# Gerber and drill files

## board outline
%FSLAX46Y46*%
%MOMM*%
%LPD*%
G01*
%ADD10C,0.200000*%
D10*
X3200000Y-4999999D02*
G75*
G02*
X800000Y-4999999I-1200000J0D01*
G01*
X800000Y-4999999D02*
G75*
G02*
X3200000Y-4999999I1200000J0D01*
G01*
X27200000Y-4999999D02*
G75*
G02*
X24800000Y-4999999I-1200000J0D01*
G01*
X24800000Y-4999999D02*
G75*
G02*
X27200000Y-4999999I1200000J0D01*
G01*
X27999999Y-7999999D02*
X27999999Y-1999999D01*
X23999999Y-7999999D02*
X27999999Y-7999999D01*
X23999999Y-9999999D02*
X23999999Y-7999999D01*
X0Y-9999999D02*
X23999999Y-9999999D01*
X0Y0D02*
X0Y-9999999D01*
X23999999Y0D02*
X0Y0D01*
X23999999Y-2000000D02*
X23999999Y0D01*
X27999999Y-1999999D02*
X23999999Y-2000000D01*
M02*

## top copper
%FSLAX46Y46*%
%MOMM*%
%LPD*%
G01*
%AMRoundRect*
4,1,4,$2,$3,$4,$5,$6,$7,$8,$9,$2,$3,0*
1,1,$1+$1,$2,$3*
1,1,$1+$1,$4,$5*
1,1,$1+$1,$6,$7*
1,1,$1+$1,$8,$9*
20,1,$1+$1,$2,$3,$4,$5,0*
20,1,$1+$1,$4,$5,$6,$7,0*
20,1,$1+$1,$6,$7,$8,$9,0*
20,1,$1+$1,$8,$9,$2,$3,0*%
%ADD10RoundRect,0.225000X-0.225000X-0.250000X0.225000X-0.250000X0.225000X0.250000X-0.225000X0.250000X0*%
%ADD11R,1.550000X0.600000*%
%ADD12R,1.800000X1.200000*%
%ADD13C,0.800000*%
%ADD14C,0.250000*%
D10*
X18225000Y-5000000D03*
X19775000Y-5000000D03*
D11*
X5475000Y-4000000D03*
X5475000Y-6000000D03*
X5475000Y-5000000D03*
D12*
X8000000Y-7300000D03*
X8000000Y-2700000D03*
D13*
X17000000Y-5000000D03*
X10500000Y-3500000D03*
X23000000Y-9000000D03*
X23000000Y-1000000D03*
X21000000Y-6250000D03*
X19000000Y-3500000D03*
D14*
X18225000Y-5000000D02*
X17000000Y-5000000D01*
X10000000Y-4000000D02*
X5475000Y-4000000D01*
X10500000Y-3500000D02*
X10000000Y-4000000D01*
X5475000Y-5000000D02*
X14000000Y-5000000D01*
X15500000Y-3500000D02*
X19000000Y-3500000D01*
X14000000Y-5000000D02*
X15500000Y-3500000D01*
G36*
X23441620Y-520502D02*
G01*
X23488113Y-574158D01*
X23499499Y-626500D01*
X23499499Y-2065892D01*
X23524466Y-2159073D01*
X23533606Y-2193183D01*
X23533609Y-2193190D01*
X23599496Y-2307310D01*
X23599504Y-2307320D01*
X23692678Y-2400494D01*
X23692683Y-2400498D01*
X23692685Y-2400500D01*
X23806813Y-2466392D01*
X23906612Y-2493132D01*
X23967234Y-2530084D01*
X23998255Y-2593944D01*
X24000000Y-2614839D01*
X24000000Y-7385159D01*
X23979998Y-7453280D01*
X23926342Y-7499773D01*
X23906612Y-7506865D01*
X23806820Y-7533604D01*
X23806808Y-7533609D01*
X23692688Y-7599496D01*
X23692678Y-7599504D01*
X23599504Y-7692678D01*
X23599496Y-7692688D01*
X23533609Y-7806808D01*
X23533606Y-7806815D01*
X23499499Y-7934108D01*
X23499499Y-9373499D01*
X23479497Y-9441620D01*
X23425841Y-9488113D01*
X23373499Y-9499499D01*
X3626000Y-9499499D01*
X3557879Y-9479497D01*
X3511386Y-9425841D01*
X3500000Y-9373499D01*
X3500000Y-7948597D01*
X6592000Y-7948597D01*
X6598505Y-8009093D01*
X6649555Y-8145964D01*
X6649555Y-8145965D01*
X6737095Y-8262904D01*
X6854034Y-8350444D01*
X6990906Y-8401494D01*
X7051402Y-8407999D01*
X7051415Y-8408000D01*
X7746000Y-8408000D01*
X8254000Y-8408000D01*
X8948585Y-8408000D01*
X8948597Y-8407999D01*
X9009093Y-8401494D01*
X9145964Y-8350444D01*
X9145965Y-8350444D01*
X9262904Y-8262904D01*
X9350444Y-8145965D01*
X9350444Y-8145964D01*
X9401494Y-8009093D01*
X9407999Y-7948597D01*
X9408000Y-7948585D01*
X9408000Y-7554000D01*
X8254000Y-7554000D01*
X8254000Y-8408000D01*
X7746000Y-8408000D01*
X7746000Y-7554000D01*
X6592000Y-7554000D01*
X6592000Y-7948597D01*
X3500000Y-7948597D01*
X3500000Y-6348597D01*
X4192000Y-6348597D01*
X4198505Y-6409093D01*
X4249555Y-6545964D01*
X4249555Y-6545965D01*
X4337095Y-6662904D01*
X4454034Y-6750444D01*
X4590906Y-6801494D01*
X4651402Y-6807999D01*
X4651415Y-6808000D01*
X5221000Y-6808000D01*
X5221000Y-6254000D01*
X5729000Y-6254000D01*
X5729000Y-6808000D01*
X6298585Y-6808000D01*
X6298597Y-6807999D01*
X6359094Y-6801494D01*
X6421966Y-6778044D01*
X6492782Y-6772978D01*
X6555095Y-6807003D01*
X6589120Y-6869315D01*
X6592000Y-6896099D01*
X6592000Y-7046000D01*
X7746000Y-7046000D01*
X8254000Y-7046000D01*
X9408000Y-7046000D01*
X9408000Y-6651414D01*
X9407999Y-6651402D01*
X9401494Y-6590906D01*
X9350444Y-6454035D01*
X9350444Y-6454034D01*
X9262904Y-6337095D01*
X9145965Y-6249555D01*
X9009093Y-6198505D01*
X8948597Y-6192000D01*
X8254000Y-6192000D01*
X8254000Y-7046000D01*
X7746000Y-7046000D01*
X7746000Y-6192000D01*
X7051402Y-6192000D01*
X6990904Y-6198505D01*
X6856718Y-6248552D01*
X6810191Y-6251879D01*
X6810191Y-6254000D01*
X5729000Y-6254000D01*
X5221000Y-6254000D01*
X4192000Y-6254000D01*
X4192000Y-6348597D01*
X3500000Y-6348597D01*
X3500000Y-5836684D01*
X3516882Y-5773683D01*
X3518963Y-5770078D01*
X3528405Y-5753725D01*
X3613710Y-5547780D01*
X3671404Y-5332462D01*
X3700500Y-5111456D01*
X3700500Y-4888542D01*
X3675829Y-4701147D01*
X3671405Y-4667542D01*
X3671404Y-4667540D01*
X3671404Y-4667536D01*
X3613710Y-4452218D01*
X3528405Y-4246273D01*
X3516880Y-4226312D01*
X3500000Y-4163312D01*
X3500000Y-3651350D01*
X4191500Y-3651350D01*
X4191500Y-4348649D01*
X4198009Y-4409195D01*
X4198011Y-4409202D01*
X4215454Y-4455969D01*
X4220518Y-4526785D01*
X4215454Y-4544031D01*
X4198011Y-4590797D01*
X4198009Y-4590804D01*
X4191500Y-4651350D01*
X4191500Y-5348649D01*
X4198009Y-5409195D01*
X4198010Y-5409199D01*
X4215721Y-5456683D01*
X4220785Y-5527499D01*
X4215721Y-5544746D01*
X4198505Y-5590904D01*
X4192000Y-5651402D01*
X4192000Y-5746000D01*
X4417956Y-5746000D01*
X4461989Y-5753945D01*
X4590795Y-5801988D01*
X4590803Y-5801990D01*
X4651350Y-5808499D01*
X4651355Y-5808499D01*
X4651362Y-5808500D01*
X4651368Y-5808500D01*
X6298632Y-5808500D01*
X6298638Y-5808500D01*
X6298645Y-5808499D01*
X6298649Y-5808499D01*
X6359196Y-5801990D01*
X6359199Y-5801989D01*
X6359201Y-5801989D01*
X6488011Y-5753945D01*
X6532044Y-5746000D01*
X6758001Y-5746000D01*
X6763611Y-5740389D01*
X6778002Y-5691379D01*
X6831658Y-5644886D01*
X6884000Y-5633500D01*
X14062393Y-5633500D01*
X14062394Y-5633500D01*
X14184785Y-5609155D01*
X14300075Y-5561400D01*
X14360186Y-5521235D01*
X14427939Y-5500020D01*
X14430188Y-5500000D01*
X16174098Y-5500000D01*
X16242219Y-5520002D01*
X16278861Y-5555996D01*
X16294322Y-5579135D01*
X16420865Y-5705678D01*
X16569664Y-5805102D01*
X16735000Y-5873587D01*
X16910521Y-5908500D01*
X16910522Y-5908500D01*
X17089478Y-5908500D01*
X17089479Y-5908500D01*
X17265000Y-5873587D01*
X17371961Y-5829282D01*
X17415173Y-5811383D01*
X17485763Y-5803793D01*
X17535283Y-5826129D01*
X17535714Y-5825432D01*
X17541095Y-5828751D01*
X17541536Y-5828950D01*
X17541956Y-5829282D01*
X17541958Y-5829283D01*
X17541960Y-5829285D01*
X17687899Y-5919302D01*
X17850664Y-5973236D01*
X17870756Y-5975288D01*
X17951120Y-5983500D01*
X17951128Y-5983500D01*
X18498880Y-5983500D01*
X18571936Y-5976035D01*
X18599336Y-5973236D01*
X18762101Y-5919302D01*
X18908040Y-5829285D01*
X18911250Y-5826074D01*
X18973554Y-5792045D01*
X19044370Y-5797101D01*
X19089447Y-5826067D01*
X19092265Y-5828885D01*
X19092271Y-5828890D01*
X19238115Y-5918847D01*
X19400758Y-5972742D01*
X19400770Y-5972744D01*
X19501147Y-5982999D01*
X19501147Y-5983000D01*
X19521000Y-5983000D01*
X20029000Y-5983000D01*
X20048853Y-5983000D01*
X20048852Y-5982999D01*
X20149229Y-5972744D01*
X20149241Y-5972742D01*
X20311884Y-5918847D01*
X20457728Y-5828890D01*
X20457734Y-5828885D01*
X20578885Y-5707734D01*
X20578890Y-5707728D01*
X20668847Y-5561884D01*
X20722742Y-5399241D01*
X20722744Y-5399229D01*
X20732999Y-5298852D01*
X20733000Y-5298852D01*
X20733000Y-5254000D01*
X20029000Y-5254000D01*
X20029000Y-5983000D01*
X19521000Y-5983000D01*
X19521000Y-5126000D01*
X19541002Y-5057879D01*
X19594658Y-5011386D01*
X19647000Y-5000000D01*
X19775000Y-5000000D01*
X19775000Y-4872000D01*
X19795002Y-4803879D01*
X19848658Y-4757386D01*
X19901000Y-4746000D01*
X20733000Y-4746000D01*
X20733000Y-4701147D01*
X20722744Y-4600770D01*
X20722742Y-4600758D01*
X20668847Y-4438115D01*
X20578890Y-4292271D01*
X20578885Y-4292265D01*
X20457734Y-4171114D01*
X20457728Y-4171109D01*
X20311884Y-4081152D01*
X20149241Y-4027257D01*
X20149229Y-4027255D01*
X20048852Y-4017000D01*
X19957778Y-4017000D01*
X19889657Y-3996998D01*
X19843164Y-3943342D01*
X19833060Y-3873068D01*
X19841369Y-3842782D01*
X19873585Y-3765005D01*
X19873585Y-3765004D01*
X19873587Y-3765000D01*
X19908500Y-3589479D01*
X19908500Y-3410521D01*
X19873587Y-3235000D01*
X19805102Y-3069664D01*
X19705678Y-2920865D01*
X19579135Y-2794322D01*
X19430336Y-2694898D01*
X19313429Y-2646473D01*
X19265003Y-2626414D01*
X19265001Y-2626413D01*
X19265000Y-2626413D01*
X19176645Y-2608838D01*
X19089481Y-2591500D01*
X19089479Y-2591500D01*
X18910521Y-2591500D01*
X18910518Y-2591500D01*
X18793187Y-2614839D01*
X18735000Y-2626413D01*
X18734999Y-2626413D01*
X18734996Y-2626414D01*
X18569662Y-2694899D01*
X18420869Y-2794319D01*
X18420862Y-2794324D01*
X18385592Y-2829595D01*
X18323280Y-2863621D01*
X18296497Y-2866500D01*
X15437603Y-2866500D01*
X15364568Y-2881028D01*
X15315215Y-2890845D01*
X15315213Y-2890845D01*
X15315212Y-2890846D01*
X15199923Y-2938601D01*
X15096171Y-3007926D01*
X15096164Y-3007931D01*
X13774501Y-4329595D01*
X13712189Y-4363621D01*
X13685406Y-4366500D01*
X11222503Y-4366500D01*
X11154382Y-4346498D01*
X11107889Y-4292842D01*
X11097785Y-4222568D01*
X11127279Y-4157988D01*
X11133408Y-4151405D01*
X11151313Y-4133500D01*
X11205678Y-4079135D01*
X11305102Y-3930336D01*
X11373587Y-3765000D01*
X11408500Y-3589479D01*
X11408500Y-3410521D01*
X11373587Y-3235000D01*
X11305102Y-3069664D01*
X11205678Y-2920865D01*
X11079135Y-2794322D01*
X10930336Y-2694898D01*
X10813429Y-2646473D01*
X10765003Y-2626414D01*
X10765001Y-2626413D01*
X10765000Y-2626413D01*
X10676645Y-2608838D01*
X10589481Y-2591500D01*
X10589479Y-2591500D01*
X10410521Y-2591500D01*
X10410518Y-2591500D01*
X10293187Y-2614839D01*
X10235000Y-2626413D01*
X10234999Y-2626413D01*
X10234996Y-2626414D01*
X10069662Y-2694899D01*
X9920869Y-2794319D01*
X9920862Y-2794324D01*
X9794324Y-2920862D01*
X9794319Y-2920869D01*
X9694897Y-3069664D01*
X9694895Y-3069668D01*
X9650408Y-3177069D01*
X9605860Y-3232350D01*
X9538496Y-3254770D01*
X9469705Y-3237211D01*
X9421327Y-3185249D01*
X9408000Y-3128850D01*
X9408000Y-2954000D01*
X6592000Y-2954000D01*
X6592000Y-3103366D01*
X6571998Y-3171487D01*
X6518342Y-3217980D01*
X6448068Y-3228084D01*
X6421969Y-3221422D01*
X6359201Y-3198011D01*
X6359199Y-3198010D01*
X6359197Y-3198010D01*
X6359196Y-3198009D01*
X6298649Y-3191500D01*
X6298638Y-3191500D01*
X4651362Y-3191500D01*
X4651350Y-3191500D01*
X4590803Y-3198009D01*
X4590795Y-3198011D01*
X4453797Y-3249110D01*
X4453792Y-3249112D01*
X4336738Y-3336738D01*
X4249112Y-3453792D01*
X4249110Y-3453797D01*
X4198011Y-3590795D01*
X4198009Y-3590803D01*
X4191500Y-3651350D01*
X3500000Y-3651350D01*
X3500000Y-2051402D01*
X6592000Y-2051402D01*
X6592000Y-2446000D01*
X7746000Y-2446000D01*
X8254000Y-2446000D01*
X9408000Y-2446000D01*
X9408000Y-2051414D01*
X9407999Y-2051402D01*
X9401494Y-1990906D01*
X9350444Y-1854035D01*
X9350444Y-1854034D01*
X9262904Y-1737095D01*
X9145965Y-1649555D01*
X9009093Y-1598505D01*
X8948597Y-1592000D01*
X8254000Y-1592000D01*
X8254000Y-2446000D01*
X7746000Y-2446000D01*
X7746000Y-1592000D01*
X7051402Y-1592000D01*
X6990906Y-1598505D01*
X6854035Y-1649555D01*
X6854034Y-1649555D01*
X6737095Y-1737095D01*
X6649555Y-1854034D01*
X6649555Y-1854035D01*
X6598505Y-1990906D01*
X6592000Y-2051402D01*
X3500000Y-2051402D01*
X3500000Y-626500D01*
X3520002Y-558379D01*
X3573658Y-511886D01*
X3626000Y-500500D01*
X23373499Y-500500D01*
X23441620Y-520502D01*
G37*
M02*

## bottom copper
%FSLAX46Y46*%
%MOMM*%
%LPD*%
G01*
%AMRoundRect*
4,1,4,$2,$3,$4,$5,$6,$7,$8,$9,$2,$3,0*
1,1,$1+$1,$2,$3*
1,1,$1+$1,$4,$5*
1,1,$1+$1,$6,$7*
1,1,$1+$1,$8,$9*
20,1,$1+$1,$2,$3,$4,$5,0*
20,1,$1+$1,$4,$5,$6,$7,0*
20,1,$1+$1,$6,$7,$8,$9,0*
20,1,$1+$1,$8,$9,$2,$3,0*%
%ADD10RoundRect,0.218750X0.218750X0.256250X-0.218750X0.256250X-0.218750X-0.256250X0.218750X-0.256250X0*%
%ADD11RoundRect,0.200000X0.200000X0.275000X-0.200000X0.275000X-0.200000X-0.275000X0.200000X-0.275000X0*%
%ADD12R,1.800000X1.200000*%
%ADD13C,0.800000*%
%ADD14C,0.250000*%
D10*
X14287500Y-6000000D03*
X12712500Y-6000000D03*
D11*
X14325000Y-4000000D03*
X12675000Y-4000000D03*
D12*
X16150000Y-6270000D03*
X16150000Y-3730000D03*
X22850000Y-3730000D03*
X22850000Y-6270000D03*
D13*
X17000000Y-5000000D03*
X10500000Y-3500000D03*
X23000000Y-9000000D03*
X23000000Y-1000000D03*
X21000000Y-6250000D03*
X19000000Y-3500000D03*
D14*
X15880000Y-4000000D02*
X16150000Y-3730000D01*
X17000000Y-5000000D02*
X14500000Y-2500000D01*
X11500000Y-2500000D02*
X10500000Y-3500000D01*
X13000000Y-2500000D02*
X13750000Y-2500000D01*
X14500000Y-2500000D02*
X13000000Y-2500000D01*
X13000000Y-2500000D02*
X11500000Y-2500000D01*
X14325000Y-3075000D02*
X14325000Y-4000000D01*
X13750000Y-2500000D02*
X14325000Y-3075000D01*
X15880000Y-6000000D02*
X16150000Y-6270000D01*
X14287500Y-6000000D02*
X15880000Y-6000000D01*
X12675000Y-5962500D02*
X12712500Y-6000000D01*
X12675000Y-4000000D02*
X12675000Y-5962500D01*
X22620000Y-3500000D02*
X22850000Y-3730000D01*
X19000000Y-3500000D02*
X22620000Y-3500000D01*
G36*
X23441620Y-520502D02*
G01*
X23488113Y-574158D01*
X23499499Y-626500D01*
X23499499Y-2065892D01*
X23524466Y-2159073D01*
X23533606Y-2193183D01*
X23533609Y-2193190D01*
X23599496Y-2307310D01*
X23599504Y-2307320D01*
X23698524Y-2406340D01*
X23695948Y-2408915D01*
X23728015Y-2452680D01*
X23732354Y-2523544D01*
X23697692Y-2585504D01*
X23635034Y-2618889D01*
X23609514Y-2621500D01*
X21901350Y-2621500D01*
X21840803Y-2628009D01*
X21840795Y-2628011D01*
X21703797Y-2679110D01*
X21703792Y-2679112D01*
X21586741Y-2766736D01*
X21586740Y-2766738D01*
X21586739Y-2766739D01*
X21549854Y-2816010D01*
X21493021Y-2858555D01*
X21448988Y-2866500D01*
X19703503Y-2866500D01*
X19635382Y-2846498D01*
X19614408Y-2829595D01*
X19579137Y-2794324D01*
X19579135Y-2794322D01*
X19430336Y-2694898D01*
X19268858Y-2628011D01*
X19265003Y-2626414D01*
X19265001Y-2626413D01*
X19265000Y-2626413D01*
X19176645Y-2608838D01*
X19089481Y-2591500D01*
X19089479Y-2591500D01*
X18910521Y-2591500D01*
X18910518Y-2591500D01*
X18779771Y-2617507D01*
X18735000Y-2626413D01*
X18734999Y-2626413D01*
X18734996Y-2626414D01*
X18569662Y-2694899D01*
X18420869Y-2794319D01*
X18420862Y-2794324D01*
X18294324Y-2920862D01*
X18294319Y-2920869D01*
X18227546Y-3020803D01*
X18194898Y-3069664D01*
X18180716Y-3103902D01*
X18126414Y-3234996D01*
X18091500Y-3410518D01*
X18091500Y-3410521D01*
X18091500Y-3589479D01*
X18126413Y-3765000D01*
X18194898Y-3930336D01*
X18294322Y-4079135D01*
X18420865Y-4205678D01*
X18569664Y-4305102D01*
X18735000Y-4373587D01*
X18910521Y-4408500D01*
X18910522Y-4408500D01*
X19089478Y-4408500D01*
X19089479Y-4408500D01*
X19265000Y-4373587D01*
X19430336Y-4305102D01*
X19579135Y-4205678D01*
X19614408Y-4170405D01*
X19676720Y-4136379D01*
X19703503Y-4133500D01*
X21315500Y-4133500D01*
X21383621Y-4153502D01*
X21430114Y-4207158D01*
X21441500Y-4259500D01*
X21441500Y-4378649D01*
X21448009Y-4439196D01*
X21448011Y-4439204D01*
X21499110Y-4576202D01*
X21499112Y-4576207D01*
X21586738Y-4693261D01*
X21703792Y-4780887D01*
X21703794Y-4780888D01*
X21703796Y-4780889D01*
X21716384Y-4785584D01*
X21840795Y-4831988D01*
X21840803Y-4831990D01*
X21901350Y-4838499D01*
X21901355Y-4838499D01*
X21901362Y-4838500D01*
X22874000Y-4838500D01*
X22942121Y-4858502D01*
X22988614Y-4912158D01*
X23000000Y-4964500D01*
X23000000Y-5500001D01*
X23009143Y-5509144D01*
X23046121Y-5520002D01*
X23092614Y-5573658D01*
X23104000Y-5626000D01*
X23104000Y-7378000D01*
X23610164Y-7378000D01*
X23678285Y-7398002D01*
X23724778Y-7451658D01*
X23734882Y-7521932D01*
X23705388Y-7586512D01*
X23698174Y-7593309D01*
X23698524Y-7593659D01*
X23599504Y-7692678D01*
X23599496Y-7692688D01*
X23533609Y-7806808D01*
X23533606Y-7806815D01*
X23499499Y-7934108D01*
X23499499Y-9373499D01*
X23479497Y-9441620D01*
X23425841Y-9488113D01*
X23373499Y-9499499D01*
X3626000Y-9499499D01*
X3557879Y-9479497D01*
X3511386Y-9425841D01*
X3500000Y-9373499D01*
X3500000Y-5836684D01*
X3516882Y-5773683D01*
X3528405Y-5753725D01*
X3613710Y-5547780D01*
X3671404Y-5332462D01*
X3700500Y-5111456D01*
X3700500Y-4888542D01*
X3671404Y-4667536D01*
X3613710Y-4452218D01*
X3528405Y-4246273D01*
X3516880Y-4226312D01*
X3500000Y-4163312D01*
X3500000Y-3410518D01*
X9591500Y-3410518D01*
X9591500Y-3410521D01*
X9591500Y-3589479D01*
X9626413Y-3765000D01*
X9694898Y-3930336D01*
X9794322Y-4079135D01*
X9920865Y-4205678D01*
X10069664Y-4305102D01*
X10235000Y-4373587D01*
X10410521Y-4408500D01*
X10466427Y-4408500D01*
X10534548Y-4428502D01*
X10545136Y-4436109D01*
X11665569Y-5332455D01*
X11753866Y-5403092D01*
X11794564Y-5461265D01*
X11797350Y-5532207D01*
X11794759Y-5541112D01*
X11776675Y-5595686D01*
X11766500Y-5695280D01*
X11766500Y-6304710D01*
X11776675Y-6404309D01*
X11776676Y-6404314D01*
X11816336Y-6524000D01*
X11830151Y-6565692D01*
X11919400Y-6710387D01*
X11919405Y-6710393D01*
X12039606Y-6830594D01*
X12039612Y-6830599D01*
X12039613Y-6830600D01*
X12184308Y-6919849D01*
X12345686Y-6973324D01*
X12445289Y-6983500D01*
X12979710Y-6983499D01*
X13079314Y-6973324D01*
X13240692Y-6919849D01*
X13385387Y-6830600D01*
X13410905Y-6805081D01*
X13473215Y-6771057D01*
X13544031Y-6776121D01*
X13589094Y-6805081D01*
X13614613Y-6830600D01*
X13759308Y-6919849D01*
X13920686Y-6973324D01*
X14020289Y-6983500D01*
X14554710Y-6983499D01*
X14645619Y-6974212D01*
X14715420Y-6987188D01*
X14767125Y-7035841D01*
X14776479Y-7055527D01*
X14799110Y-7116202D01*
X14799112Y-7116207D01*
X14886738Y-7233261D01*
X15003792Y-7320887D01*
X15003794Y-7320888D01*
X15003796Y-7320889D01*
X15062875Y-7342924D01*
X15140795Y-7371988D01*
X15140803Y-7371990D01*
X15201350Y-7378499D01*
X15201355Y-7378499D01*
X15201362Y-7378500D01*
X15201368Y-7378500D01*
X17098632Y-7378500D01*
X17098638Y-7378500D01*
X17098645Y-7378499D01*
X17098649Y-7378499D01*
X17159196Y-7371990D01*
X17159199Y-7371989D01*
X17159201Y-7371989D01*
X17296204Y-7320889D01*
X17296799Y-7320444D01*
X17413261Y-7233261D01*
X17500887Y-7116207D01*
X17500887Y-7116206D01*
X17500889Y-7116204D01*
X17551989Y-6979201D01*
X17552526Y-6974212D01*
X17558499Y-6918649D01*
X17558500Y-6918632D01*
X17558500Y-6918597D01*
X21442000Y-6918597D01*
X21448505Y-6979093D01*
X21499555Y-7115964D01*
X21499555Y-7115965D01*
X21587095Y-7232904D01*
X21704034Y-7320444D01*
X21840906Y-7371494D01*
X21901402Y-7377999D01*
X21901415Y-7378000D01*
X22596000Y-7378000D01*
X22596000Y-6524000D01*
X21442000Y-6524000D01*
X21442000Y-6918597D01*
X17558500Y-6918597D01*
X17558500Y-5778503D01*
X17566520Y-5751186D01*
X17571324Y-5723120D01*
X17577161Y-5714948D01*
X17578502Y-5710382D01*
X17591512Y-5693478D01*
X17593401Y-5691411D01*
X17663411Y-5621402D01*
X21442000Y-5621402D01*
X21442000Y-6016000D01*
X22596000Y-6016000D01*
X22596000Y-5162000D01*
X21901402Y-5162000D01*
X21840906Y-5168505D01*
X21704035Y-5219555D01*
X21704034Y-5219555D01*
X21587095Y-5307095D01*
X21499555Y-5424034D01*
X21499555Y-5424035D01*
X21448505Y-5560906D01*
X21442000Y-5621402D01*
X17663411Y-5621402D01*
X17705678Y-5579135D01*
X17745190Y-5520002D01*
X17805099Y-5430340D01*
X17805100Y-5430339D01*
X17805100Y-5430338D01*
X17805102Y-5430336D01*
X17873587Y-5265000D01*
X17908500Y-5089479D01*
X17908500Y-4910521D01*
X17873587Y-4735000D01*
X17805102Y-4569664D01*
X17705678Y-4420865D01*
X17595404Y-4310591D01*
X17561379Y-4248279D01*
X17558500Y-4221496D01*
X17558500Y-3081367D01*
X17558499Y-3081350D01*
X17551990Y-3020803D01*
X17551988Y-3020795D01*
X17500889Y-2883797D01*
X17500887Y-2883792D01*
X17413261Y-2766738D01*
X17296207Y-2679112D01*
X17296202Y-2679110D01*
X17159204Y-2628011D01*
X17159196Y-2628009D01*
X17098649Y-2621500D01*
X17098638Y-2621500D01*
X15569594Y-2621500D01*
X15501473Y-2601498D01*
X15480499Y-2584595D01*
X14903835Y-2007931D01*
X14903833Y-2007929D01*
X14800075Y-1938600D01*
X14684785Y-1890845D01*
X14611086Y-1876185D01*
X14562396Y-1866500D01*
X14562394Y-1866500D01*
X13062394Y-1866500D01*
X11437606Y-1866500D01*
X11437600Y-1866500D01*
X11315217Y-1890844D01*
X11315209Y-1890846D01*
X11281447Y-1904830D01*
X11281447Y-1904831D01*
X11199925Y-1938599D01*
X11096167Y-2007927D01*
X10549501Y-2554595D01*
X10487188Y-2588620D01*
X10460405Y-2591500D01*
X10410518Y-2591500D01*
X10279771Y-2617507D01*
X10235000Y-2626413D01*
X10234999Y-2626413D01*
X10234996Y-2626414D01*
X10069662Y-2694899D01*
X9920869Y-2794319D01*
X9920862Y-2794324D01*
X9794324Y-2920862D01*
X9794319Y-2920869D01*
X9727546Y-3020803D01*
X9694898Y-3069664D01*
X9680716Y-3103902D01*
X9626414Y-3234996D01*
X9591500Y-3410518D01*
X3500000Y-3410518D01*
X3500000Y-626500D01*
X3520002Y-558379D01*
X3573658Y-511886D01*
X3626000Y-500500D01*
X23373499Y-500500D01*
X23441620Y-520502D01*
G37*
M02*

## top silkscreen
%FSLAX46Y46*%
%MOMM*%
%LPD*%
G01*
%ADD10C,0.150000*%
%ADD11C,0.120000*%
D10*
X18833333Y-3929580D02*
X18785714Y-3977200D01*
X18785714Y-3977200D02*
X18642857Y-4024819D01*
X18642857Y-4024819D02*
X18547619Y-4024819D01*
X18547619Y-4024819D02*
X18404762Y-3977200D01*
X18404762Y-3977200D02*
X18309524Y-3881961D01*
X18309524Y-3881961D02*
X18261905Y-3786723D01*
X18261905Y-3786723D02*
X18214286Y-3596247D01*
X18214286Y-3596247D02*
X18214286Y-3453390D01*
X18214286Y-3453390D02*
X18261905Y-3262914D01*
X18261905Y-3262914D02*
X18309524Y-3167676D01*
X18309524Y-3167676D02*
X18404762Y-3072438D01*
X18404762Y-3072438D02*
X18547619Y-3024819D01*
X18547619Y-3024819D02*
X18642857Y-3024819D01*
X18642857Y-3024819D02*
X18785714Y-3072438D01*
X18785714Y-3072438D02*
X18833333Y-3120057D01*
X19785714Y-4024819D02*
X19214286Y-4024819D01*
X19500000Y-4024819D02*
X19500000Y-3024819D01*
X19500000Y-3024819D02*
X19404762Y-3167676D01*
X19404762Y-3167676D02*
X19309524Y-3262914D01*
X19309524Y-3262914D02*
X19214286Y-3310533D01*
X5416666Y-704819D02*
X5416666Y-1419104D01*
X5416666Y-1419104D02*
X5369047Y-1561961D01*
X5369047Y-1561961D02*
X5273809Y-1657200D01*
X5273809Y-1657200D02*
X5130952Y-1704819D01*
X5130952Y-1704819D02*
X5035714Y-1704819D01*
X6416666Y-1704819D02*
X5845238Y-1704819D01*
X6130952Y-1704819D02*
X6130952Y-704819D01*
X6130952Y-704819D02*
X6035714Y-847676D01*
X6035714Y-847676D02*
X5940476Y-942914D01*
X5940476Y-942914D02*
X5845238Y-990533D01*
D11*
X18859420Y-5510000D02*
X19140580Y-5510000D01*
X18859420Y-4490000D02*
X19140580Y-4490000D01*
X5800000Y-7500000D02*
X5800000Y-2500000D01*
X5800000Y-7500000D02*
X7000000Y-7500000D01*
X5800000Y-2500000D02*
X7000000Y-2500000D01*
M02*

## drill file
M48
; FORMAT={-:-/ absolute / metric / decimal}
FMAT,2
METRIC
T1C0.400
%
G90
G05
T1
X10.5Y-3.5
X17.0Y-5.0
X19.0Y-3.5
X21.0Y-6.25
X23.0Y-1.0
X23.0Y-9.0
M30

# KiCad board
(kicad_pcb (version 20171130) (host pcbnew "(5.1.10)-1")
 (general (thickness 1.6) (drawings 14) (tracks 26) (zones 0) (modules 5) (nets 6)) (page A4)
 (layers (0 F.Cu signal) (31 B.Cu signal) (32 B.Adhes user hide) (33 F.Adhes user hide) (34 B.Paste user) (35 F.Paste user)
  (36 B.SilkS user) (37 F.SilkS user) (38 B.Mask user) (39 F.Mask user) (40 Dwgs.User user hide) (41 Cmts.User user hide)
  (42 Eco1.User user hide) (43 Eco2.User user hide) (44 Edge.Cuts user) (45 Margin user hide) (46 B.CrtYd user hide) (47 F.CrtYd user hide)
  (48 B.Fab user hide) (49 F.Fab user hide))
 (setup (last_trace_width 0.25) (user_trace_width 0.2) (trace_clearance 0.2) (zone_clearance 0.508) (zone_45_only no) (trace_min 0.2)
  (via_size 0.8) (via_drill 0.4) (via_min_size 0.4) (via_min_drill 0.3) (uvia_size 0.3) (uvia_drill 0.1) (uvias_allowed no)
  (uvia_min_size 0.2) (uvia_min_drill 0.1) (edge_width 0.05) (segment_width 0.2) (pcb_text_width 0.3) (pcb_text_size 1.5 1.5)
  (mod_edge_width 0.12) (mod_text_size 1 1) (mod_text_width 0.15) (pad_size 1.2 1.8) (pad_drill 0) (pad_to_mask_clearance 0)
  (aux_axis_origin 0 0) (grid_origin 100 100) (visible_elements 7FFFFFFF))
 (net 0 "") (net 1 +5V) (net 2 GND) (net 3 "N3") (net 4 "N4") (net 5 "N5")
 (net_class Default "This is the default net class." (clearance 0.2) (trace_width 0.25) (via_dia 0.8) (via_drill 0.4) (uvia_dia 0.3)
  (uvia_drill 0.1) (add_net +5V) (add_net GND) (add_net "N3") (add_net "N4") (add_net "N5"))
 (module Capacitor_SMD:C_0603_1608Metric (layer F.Cu) (at 19 5)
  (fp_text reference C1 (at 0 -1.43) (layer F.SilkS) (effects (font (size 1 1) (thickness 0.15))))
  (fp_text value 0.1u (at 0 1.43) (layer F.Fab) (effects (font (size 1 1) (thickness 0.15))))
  (fp_line (start -0.14058 0.51) (end 0.14058 0.51) (layer F.SilkS) (width 0.12))
  (fp_line (start -0.14058 -0.51) (end 0.14058 -0.51) (layer F.SilkS) (width 0.12))
  (pad 1 smd roundrect (at -0.775 0) (size 0.9 0.95) (layers F.Cu F.Paste F.Mask) (roundrect_rratio 0.25) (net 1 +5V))
  (pad 2 smd roundrect (at 0.775 0) (size 0.9 0.95) (layers F.Cu F.Paste F.Mask) (roundrect_rratio 0.25) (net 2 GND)))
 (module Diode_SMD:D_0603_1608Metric (layer B.Cu) (at 13.5 6 180)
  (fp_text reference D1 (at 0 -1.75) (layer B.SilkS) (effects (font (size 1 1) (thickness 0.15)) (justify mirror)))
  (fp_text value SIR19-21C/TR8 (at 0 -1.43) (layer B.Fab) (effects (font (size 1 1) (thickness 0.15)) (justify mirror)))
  (pad 1 smd roundrect (at -0.7875 0 180) (size 0.875 0.95) (layers B.Cu B.Paste B.Mask) (roundrect_rratio 0.25) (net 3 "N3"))
  (pad 2 smd roundrect (at 0.7875 0 180) (size 0.875 0.95) (layers B.Cu B.Paste B.Mask) (roundrect_rratio 0.25) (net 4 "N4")))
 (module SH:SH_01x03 (layer F.Cu) (at 8 5 90)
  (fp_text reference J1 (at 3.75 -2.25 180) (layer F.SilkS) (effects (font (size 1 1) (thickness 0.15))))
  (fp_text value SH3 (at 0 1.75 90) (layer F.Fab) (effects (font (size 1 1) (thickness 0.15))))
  (fp_line (start -2.5 -2.2) (end 2.5 -2.2) (layer F.SilkS) (width 0.12))
  (fp_line (start -2.5 -2.2) (end -2.5 -1) (layer F.SilkS) (width 0.12))
  (fp_line (start 2.5 -2.2) (end 2.5 -1) (layer F.SilkS) (width 0.12))
  (pad 3 smd rect (at 1 -2.525 90) (size 0.6 1.55) (layers F.Cu F.Paste F.Mask) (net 1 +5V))
  (pad 1 smd rect (at -1 -2.525 90) (size 0.6 1.55) (layers F.Cu F.Paste F.Mask) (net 2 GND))
  (pad 2 smd rect (at 0 -2.525 90) (size 0.6 1.55) (layers F.Cu F.Paste F.Mask) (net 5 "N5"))
  (pad MP smd rect (at -2.3 0 90) (size 1.2 1.8) (layers F.Cu F.Paste F.Mask) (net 2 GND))
  (pad MP smd rect (at 2.3 0 90) (size 1.2 1.8) (layers F.Cu F.Paste F.Mask) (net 2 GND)))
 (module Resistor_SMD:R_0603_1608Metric (layer B.Cu) (at 13.5 4 180)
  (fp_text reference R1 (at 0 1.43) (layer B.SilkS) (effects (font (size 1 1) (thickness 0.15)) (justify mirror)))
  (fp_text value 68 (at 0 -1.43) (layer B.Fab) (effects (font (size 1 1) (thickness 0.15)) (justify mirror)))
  (pad 1 smd roundrect (at -0.825 0 180) (size 0.8 0.95) (layers B.Cu B.Paste B.Mask) (roundrect_rratio 0.25) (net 1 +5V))
  (pad 2 smd roundrect (at 0.825 0 180) (size 0.8 0.95) (layers B.Cu B.Paste B.Mask) (roundrect_rratio 0.25) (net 4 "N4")))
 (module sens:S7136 (layer B.Cu) (at 19.5 5)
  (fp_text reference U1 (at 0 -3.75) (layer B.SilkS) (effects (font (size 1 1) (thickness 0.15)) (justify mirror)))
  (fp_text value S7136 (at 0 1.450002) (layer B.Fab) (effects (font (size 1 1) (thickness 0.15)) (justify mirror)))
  (pad 1 smd rect (at -3.35 1.27) (size 1.8 1.2) (layers B.Cu B.Paste B.Mask) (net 3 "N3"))
  (pad 2 smd rect (at -3.35 -1.27) (size 1.8 1.2) (layers B.Cu B.Paste B.Mask) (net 1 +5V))
  (pad 3 smd rect (at 3.35 -1.27) (size 1.8 1.2) (layers B.Cu B.Paste B.Mask) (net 5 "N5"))
  (pad 4 smd rect (at 3.35 1.27) (size 1.8 1.2) (layers B.Cu B.Paste B.Mask) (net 2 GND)))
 (gr_circle (center 2 4.999999) (end 3.2 4.999999) (layer Edge.Cuts) (width 0.2))
 (gr_circle (center 26 4.999999) (end 27.2 4.999999) (layer Edge.Cuts) (width 0.2))
 (gr_line (start 27.999999 7.999999) (end 27.999999 1.999999) (layer Edge.Cuts) (width 0.2))
 (gr_line (start 23.999999 7.999999) (end 27.999999 7.999999) (layer Edge.Cuts) (width 0.2))
 (gr_line (start 23.999999 9.999999) (end 23.999999 7.999999) (layer Edge.Cuts) (width 0.2))
 (gr_line (start 0 9.999999) (end 23.999999 9.999999) (layer Edge.Cuts) (width 0.2))
 (gr_line (start 0 0) (end 0 9.999999) (layer Edge.Cuts) (width 0.2))
 (gr_line (start 23.999999 0) (end 0 0) (layer Edge.Cuts) (width 0.2))
 (gr_line (start 23.999999 2) (end 23.999999 0) (layer Edge.Cuts) (width 0.2))
 (gr_line (start 27.999999 1.999999) (end 23.999999 2) (layer Edge.Cuts) (width 0.2))
 (segment (start 15.88 4) (end 16.15 3.73) (width 0.25) (layer B.Cu) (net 1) (status 30))
 (via (at 17 5) (size 0.8) (drill 0.4) (layers F.Cu B.Cu) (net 1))
 (segment (start 18.225 5) (end 17 5) (width 0.25) (layer F.Cu) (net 1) (status 10))
 (segment (start 17 5) (end 14.5 2.5) (width 0.25) (layer B.Cu) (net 1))
 (via (at 10.5 3.5) (size 0.8) (drill 0.4) (layers F.Cu B.Cu) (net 1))
 (segment (start 11.5 2.5) (end 10.5 3.5) (width 0.25) (layer B.Cu) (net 1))
 (segment (start 10 4) (end 5.475 4) (width 0.25) (layer F.Cu) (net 1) (status 20))
 (segment (start 10.5 3.5) (end 10 4) (width 0.25) (layer F.Cu) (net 1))
 (segment (start 13 2.5) (end 13.75 2.5) (width 0.25) (layer B.Cu) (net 1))
 (segment (start 14.5 2.5) (end 13 2.5) (width 0.25) (layer B.Cu) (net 1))
 (segment (start 13 2.5) (end 11.5 2.5) (width 0.25) (layer B.Cu) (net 1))
 (segment (start 14.325 3.075) (end 14.325 4) (width 0.25) (layer B.Cu) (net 1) (status 20))
 (segment (start 13.75 2.5) (end 14.325 3.075) (width 0.25) (layer B.Cu) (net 1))
 (via (at 23 9) (size 0.8) (drill 0.4) (layers F.Cu B.Cu) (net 2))
 (via (at 23 1) (size 0.8) (drill 0.4) (layers F.Cu B.Cu) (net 2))
 (via (at 21 6.25) (size 0.8) (drill 0.4) (layers F.Cu B.Cu) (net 2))
 (segment (start 15.88 6) (end 16.15 6.27) (width 0.25) (layer B.Cu) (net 3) (status 30))
 (segment (start 14.2875 6) (end 15.88 6) (width 0.25) (layer B.Cu) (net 3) (status 30))
 (segment (start 12.675 5.9625) (end 12.7125 6) (width 0.25) (layer B.Cu) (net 4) (status 30))
 (segment (start 12.675 4) (end 12.675 5.9625) (width 0.25) (layer B.Cu) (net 4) (status 30))
 (segment (start 5.475 5) (end 14 5) (width 0.25) (layer F.Cu) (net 5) (status 10))
 (via (at 19 3.5) (size 0.8) (drill 0.4) (layers F.Cu B.Cu) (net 5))
 (segment (start 15.5 3.5) (end 19 3.5) (width 0.25) (layer F.Cu) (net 5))
 (segment (start 14 5) (end 15.5 3.5) (width 0.25) (layer F.Cu) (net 5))
 (segment (start 22.62 3.5) (end 22.85 3.73) (width 0.25) (layer B.Cu) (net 5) (status 30))
 (segment (start 19 3.5) (end 22.62 3.5) (width 0.25) (layer B.Cu) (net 5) (status 20))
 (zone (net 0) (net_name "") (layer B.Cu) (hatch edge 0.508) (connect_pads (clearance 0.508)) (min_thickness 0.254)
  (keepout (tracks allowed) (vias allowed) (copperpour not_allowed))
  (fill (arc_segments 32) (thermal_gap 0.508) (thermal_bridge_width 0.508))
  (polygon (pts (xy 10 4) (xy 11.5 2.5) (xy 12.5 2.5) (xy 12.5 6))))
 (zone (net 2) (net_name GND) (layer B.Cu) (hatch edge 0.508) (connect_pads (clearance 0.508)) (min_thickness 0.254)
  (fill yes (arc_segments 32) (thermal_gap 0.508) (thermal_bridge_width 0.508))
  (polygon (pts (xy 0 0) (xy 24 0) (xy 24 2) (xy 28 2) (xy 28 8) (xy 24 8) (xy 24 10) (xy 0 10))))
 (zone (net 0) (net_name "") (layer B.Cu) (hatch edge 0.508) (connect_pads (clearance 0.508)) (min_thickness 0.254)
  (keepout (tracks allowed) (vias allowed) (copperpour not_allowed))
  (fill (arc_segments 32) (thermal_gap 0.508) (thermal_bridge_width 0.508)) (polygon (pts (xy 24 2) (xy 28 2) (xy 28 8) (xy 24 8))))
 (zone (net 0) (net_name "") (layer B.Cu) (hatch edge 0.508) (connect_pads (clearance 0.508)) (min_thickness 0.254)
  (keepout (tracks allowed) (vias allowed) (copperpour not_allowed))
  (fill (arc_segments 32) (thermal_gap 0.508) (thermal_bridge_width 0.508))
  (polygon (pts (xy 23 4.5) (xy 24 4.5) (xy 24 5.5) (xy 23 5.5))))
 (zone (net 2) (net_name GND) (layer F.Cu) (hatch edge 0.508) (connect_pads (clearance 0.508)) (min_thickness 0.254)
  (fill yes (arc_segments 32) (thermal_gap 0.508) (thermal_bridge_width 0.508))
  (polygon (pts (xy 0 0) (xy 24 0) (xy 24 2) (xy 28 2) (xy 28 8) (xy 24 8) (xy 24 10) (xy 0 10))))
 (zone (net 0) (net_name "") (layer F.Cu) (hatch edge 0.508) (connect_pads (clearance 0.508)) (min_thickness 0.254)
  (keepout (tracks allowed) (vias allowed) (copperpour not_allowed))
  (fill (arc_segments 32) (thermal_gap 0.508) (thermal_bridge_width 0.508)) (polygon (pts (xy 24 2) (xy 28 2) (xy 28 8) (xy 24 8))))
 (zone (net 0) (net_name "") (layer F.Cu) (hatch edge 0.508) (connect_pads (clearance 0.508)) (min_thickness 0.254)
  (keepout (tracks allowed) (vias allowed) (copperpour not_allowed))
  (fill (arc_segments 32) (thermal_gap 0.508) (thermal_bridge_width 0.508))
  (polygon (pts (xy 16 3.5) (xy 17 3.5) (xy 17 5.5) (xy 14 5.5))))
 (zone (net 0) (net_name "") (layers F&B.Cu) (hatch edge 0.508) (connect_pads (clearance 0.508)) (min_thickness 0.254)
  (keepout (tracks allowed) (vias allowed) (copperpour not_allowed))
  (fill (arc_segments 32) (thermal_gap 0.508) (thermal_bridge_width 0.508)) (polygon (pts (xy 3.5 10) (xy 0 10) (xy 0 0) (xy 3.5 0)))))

